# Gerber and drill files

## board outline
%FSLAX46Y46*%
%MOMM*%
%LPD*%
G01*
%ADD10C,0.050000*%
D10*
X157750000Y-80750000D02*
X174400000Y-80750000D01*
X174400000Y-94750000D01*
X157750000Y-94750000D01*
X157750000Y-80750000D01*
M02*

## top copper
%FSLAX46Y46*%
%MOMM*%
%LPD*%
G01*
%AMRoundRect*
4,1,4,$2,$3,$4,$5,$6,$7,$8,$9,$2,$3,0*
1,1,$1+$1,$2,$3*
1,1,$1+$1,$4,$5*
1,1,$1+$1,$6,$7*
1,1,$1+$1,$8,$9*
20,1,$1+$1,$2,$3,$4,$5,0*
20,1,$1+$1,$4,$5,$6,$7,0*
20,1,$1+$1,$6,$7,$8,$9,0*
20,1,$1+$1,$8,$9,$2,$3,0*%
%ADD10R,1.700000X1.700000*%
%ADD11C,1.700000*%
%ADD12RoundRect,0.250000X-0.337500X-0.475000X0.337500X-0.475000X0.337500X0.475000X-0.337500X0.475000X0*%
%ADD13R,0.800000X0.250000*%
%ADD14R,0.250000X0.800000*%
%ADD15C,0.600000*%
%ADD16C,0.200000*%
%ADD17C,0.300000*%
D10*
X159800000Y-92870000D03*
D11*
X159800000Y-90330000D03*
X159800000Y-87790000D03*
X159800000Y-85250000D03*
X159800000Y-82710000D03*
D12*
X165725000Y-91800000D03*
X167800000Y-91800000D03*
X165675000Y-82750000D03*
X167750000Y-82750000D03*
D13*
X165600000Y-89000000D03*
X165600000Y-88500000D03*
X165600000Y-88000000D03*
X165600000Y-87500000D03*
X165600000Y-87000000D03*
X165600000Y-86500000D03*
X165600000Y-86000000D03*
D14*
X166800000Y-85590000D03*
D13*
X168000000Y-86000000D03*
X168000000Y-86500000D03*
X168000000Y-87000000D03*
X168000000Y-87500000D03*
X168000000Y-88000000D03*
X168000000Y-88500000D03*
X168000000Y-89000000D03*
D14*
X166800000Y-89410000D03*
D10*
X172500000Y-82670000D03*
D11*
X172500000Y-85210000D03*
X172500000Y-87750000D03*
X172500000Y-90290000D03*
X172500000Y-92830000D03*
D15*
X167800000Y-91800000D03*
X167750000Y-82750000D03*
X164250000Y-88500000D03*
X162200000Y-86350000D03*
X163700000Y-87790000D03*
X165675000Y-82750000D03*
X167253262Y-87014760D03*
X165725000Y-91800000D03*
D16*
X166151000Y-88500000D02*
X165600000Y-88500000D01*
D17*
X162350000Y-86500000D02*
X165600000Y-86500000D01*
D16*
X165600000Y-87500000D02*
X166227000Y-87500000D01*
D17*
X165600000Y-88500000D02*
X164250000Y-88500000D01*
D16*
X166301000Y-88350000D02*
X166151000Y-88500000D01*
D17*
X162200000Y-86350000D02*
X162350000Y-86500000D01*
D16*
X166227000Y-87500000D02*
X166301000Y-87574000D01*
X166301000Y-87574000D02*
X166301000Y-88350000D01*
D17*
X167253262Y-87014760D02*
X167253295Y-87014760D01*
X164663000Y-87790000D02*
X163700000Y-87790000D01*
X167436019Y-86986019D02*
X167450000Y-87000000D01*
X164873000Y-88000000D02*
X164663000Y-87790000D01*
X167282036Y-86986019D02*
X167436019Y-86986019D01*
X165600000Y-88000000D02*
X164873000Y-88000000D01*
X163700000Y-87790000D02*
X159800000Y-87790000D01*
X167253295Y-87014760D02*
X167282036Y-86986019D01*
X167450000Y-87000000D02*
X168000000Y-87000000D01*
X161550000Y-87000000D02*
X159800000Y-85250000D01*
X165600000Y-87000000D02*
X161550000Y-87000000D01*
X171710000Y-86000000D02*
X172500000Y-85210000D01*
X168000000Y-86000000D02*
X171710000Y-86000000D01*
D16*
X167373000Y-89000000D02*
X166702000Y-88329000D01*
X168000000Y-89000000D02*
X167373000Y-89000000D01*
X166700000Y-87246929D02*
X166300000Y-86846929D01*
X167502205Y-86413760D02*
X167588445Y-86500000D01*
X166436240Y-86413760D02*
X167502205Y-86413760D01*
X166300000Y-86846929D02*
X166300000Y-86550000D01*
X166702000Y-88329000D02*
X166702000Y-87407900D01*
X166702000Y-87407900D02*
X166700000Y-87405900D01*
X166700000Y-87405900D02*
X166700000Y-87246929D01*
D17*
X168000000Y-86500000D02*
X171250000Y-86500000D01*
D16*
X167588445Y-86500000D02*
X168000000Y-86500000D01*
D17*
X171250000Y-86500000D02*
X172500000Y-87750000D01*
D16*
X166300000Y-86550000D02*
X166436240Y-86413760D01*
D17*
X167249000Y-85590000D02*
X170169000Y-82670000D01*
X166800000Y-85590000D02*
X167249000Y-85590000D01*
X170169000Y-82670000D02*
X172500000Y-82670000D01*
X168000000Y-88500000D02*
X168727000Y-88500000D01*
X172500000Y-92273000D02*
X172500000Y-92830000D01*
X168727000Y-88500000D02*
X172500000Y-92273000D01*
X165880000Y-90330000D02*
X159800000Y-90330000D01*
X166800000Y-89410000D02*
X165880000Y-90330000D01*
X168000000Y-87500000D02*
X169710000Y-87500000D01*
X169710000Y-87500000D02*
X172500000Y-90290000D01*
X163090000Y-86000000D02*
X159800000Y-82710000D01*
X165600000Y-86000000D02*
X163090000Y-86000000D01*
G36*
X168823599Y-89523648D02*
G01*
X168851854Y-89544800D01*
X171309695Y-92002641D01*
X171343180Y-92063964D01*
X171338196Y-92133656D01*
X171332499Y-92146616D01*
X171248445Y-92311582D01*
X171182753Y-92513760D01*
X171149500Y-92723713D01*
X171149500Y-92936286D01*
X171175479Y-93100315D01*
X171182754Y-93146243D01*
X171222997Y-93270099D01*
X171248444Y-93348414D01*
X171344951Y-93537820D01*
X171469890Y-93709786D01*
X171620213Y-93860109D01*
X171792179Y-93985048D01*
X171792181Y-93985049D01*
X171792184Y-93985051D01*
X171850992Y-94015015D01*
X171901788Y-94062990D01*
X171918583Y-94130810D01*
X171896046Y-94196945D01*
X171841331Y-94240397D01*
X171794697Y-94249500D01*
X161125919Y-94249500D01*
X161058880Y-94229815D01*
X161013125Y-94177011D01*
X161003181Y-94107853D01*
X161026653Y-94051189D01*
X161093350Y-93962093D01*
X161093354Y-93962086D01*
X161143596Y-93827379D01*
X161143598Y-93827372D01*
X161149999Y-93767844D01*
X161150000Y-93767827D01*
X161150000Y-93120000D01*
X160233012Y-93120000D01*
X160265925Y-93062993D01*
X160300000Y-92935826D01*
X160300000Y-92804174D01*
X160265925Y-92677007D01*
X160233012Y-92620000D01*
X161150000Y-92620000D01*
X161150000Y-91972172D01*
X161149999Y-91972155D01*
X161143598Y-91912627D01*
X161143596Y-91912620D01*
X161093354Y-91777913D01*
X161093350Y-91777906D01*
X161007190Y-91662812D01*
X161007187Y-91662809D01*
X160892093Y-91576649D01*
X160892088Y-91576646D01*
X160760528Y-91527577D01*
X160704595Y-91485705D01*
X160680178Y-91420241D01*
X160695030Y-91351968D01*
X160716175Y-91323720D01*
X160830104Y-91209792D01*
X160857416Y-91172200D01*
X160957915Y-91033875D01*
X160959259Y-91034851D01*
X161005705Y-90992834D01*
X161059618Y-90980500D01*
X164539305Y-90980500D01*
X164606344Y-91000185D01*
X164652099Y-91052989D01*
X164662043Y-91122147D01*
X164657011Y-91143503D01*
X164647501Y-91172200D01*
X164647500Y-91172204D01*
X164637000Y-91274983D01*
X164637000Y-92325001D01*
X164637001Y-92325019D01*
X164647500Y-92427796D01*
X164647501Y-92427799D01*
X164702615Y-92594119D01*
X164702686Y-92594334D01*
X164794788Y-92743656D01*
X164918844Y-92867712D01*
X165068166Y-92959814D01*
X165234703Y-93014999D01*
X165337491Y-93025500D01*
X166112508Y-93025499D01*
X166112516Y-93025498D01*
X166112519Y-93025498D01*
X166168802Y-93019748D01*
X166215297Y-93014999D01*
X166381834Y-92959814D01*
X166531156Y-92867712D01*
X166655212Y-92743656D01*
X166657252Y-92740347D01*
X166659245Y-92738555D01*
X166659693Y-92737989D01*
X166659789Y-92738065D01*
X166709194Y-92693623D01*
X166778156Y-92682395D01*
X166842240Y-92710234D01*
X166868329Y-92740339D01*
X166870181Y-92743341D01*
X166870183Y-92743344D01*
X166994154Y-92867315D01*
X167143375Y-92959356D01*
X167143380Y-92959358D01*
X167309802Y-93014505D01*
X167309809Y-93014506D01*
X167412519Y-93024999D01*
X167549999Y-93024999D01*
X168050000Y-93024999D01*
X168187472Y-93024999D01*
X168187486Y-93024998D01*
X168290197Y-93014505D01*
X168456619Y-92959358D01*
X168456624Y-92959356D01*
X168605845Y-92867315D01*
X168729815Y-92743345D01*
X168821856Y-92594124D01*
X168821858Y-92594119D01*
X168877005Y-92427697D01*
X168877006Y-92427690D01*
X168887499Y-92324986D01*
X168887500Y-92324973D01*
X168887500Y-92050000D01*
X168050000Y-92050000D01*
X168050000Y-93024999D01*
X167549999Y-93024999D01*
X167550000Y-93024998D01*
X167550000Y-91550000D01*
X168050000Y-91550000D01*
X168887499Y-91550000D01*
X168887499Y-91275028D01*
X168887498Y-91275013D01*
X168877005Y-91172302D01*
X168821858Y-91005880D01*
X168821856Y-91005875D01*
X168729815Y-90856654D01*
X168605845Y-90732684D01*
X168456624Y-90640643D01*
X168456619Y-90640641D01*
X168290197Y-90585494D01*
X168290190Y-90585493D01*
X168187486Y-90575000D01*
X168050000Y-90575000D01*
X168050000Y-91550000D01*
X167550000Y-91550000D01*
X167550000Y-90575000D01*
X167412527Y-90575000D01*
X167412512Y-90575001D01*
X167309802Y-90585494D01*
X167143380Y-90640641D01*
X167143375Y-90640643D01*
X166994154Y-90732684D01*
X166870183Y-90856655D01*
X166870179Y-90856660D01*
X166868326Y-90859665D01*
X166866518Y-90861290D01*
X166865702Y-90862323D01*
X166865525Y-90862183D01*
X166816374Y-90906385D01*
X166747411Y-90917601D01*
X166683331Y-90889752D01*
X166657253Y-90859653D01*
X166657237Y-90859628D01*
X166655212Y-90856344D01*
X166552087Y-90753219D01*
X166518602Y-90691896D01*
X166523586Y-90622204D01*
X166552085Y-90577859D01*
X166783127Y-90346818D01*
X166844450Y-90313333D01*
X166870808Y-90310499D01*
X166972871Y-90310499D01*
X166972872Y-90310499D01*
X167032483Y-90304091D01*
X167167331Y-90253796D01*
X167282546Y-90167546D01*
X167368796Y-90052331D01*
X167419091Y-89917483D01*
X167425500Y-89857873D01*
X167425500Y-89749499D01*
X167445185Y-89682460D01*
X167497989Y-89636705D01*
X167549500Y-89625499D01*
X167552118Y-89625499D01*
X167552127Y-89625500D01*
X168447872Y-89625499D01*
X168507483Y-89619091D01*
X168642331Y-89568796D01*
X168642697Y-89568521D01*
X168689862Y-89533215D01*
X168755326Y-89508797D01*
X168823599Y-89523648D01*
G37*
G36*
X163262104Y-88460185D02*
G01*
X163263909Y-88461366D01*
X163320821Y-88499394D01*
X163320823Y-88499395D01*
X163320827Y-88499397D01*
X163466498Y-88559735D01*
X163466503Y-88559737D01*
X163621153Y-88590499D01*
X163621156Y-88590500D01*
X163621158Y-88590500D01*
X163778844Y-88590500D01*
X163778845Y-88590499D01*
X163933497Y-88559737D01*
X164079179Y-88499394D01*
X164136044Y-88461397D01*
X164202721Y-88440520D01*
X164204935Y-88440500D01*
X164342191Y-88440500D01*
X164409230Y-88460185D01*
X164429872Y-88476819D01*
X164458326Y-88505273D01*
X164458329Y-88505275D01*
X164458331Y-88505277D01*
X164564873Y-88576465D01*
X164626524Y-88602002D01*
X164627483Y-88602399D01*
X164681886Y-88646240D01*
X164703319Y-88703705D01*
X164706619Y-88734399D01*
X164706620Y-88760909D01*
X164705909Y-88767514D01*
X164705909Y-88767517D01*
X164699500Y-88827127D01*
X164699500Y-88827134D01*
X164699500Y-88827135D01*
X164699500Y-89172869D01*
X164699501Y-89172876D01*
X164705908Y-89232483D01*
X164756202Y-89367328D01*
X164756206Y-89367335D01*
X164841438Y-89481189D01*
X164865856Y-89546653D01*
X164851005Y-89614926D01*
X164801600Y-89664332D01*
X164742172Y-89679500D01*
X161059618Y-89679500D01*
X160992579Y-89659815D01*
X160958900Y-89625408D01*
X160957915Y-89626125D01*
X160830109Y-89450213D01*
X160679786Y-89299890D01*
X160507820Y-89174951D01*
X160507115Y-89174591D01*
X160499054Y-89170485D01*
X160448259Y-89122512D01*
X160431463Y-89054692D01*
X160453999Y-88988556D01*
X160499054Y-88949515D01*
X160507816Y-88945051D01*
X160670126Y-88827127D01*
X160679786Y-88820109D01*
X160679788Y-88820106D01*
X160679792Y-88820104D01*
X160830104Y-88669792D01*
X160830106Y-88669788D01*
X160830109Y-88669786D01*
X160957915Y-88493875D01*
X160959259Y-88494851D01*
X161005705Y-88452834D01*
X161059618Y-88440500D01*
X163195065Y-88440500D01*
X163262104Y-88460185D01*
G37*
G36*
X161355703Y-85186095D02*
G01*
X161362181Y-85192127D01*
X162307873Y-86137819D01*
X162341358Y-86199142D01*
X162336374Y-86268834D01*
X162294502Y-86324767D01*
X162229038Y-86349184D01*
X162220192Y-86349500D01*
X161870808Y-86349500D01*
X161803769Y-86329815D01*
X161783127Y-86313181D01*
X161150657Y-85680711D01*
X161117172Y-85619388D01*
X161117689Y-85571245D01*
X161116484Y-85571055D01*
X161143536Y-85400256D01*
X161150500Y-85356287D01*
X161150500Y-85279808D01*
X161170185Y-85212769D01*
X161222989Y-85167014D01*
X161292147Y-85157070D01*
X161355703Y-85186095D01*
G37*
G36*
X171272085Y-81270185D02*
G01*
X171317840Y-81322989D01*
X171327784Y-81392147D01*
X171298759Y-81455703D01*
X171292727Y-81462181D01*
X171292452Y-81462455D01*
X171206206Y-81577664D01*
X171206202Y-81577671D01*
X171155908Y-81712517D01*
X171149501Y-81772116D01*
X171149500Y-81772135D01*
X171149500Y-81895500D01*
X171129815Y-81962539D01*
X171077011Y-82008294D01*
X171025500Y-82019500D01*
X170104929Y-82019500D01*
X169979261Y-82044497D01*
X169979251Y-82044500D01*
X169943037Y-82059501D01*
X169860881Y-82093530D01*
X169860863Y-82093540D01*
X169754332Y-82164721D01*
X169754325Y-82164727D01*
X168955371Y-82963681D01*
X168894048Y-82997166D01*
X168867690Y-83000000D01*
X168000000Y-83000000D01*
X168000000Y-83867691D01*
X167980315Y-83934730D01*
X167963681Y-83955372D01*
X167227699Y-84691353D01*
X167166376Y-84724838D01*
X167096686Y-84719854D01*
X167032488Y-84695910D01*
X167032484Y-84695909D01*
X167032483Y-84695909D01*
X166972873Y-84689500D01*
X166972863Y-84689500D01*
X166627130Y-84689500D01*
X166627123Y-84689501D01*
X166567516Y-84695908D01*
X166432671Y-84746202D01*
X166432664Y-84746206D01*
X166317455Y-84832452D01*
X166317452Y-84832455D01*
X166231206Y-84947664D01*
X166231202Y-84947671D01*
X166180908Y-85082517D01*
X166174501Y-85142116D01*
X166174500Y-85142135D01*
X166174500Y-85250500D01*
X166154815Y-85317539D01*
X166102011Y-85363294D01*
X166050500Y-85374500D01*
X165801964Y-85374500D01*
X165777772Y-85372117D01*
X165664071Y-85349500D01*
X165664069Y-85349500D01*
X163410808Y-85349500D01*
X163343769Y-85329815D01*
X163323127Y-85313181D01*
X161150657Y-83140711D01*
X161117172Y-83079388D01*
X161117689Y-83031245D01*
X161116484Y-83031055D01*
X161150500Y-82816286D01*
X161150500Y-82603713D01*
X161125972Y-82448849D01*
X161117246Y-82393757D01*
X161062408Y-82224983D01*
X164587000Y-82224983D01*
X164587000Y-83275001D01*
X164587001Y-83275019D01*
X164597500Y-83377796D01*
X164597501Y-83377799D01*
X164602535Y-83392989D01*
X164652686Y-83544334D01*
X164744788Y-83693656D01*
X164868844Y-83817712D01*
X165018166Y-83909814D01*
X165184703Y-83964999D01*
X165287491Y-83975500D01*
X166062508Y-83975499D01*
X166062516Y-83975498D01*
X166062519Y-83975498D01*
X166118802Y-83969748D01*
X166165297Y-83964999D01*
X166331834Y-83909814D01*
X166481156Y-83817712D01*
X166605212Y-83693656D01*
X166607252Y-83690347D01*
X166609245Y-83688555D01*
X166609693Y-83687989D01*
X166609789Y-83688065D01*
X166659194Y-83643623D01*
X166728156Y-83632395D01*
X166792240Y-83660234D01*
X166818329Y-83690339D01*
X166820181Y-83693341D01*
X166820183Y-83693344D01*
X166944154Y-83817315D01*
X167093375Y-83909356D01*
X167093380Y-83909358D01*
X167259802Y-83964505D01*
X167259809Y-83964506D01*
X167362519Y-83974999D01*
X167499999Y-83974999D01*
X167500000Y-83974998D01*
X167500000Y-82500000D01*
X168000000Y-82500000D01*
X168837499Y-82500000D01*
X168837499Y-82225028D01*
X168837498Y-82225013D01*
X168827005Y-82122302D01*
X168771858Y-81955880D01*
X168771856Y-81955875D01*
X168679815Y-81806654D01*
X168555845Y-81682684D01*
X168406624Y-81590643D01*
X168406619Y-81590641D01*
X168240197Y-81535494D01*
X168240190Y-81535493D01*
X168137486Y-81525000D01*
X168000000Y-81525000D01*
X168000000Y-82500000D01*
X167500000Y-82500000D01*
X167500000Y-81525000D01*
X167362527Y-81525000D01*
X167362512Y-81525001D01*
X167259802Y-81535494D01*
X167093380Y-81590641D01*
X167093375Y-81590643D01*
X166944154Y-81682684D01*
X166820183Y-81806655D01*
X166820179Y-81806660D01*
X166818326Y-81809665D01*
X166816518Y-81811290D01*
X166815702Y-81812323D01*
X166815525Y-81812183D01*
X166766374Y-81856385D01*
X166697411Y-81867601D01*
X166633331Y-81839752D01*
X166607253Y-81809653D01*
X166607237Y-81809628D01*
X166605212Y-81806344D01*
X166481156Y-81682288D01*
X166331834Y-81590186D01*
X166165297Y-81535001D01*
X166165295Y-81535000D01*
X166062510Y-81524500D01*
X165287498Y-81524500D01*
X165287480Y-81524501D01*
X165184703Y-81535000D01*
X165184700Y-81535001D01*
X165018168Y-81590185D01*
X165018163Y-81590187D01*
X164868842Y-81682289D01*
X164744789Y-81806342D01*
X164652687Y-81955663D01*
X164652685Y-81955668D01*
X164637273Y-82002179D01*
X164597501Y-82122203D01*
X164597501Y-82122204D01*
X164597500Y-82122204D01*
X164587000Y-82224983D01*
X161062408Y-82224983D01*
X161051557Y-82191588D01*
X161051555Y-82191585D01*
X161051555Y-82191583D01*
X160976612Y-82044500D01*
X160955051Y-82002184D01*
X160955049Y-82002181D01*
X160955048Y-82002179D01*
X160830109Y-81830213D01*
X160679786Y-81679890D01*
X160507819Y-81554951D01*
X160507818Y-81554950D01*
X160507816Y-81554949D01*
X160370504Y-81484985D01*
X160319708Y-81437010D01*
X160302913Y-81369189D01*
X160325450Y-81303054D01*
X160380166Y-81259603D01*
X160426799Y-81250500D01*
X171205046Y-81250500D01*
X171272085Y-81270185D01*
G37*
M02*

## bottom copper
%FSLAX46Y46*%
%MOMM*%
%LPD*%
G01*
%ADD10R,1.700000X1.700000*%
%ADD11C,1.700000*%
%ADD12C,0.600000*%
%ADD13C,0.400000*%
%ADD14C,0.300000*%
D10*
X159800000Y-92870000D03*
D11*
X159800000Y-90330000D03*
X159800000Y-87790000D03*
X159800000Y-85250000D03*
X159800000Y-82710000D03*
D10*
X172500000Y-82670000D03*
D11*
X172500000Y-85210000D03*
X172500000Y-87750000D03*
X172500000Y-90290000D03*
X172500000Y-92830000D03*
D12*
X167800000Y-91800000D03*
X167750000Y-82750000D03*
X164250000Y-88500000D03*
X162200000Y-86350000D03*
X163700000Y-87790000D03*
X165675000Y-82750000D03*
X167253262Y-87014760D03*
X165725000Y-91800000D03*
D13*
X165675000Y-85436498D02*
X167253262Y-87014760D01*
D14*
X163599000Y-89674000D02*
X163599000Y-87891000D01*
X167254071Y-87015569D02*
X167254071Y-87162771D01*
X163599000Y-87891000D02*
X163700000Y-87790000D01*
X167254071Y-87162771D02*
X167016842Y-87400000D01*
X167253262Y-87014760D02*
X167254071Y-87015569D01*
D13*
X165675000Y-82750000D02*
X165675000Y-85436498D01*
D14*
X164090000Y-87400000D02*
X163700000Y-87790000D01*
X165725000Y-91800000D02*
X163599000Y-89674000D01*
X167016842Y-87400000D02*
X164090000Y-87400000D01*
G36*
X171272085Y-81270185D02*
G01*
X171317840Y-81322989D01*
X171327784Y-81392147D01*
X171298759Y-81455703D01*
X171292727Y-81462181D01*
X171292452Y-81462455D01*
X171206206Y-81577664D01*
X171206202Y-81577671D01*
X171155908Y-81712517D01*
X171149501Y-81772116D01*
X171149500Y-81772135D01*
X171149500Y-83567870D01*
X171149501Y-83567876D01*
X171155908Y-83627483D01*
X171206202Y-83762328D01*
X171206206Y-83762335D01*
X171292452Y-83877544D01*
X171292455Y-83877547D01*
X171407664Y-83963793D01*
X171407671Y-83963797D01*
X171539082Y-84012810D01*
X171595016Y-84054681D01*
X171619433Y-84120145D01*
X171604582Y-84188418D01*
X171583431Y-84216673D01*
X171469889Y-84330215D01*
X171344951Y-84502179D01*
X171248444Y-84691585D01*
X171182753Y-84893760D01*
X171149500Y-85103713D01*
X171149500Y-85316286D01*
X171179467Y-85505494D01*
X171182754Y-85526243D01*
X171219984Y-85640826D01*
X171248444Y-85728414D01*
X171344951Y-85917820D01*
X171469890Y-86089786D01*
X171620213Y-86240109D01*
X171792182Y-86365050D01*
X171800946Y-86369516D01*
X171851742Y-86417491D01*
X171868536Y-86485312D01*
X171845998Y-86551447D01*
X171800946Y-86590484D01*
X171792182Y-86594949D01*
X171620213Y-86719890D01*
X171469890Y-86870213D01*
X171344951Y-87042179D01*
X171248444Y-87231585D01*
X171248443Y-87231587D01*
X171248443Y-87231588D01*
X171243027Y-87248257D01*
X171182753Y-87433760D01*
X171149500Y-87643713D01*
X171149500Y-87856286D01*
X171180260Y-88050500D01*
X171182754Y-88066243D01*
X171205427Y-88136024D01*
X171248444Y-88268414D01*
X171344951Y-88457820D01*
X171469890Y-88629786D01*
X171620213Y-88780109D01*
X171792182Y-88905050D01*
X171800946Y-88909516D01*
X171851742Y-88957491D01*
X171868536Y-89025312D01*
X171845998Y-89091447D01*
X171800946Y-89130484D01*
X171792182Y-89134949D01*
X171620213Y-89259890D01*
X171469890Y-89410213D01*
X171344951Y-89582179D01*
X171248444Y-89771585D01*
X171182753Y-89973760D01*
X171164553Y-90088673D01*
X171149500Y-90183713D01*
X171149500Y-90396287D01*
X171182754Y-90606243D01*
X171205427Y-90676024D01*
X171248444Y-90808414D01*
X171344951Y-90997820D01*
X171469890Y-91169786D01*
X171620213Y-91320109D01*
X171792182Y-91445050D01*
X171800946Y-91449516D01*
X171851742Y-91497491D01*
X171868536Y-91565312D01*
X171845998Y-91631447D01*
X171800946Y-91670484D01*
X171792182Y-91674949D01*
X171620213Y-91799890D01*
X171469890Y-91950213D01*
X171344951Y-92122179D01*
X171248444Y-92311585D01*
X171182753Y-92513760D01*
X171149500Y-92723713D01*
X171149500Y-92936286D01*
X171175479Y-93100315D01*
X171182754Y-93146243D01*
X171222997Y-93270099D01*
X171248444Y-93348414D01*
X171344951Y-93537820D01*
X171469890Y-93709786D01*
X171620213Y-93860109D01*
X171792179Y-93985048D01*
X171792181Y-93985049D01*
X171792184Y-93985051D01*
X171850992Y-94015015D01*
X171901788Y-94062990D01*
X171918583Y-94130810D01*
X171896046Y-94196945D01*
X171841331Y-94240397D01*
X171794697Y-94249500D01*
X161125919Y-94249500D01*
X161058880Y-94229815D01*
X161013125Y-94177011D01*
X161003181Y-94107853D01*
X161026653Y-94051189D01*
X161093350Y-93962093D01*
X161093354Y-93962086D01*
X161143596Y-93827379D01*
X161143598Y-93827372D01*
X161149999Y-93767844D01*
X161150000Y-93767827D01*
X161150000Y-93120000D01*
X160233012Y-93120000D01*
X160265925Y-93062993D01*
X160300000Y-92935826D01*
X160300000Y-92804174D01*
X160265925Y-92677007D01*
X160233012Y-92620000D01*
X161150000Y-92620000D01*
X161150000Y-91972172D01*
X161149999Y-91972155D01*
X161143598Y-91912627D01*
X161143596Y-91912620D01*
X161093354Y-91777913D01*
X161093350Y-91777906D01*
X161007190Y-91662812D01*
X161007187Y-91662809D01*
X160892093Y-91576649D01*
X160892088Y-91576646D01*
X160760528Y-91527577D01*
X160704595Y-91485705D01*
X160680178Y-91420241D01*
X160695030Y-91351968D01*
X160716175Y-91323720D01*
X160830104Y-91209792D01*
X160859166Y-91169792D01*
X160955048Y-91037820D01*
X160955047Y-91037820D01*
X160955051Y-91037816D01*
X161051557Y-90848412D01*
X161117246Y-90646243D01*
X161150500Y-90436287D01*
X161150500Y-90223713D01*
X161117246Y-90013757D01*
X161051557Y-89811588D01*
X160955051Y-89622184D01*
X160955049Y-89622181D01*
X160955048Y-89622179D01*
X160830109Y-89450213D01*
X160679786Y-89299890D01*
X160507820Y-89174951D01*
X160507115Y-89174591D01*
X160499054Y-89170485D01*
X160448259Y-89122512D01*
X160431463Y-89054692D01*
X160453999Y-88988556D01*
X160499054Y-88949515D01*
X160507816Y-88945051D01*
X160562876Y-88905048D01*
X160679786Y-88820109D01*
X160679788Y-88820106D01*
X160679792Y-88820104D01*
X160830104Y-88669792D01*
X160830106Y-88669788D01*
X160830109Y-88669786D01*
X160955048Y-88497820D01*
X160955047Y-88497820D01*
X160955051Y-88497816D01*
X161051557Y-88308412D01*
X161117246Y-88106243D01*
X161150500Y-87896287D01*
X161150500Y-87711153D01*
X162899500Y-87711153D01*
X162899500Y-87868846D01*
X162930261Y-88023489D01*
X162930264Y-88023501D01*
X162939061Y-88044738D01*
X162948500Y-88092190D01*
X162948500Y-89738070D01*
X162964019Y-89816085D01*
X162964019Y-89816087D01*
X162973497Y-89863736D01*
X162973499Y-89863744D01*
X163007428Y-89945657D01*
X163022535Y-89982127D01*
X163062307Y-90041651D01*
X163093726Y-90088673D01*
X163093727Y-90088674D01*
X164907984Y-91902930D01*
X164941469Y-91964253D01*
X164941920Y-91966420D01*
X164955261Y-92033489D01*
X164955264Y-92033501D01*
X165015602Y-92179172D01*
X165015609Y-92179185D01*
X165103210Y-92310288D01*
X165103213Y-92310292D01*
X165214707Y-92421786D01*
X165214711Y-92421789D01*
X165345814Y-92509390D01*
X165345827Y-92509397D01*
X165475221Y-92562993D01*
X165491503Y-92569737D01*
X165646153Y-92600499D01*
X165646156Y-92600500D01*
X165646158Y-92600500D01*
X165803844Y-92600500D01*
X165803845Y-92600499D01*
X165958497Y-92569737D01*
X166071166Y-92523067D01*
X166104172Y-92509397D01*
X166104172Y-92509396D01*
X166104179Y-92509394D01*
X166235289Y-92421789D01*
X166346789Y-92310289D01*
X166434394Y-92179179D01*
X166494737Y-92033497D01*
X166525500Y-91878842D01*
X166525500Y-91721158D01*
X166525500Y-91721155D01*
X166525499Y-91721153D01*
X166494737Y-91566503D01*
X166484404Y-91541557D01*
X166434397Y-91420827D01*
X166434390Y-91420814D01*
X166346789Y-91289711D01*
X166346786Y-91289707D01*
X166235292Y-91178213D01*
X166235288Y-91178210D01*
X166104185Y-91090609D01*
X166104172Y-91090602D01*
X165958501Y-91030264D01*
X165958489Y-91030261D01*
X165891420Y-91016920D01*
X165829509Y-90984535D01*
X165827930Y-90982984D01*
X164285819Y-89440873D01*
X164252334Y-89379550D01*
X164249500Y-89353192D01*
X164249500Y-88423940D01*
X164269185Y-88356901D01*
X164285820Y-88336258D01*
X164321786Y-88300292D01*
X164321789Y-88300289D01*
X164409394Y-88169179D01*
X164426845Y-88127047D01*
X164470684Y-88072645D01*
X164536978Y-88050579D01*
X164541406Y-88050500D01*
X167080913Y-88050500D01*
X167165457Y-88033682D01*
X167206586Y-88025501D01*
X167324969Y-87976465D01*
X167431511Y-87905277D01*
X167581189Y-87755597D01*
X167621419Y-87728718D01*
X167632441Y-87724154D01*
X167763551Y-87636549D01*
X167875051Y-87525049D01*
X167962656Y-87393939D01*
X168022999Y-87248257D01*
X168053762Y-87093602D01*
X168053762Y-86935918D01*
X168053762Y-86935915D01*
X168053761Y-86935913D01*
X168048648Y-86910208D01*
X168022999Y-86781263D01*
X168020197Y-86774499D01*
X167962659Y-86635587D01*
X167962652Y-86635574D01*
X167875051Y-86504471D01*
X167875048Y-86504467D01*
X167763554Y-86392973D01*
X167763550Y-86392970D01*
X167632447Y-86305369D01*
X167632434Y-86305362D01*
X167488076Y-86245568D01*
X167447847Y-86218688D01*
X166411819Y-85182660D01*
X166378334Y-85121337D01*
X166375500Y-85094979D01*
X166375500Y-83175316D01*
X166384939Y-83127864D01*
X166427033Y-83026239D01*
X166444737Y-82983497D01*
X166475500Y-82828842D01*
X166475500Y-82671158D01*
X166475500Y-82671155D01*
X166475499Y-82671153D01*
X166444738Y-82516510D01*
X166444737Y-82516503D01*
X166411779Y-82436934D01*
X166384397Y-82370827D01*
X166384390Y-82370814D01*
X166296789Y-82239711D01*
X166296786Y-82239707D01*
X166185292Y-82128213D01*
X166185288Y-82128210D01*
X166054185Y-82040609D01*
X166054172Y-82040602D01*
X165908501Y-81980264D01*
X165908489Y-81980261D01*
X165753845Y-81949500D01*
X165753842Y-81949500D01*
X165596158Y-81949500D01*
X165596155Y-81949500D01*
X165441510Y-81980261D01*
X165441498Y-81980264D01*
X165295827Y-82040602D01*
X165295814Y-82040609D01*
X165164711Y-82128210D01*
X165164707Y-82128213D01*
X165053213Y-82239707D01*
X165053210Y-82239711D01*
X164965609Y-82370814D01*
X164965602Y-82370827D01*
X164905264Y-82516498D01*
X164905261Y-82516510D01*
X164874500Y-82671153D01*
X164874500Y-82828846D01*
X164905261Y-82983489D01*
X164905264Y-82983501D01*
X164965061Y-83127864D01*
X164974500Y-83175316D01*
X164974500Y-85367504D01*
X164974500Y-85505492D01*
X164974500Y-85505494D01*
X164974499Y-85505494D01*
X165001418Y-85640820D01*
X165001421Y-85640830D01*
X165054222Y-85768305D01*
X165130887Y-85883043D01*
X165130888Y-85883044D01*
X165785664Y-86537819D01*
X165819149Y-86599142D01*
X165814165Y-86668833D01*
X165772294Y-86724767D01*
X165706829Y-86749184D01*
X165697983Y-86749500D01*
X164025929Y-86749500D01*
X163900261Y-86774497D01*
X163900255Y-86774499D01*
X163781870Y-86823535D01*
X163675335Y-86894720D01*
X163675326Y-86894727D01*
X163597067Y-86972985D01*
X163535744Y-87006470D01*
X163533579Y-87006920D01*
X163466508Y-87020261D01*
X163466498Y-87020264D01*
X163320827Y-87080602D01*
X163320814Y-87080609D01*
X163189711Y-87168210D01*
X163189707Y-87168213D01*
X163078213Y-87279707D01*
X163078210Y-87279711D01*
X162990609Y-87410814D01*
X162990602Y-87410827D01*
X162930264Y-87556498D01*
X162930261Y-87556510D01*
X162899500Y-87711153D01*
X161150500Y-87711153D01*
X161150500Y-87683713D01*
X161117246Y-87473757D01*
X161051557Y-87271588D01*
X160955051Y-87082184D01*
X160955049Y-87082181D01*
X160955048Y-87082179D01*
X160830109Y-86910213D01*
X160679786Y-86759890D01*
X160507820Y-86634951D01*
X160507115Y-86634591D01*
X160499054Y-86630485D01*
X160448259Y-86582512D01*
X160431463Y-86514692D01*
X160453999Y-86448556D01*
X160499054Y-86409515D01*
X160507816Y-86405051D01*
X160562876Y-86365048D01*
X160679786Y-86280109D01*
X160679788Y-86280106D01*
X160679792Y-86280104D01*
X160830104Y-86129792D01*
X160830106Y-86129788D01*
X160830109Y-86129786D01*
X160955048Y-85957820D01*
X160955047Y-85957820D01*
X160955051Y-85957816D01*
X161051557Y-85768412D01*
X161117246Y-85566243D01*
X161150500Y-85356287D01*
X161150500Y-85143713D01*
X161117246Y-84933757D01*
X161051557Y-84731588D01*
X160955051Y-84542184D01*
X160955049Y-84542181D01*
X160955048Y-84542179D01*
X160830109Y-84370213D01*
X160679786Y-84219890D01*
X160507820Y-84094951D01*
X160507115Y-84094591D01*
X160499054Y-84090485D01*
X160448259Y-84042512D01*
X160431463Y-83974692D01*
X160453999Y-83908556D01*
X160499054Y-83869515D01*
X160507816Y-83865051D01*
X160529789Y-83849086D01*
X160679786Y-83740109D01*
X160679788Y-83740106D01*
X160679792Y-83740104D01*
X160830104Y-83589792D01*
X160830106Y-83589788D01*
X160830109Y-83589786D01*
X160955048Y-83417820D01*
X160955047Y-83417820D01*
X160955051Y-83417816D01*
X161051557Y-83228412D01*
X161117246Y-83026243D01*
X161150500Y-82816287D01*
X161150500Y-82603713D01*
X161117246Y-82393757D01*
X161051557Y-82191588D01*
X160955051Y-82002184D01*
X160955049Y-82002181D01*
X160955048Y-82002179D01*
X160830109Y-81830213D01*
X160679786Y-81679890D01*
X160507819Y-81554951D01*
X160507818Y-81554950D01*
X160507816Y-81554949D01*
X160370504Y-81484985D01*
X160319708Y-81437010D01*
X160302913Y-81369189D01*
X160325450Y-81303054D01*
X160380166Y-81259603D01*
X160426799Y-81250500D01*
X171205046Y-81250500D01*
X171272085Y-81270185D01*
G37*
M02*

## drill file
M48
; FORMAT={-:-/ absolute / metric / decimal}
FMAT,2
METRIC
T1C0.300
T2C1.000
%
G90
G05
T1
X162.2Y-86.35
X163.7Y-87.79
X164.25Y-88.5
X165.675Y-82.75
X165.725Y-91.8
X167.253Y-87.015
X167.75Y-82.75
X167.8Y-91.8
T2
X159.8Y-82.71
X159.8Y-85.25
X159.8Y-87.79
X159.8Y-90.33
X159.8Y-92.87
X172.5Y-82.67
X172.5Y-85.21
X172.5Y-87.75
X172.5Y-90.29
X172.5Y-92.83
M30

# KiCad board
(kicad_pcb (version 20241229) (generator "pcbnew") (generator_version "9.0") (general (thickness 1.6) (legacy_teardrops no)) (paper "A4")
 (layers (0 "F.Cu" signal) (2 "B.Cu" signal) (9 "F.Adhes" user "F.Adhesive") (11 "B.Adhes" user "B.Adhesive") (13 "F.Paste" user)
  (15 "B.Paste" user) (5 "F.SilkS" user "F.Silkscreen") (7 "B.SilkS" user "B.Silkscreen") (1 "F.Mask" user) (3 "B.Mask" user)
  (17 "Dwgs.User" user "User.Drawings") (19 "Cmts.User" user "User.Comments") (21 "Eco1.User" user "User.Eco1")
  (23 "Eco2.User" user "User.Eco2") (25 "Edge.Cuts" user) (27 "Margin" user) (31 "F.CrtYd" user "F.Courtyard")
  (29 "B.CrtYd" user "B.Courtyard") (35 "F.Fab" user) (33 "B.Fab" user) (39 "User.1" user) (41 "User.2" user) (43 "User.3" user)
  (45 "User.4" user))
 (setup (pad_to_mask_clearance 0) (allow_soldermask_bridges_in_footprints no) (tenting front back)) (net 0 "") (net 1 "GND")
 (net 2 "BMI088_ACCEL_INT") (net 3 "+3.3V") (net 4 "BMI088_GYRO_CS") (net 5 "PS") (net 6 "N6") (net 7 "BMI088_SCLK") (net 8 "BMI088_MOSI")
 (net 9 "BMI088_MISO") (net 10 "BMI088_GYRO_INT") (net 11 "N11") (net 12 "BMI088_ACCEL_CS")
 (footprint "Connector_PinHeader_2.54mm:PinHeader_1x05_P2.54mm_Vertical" (layer "F.Cu") (at 159.8 92.87 180)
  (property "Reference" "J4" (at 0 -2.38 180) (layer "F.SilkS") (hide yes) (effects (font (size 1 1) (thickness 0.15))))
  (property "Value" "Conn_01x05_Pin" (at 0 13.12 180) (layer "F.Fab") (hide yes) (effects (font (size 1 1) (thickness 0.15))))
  (pad "1" thru_hole rect (at 0 0 180) (size 1.7 1.7) (drill 1) (layers "*.Cu" "*.Mask") (remove_unused_layers no) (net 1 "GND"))
  (pad "2" thru_hole circle (at 0 2.54 180) (size 1.7 1.7) (drill 1) (layers "*.Cu" "*.Mask") (remove_unused_layers no)
   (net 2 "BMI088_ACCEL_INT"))
  (pad "3" thru_hole circle (at 0 5.08 180) (size 1.7 1.7) (drill 1) (layers "*.Cu" "*.Mask") (remove_unused_layers no) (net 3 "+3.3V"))
  (pad "4" thru_hole circle (at 0 7.62 180) (size 1.7 1.7) (drill 1) (layers "*.Cu" "*.Mask") (remove_unused_layers no)
   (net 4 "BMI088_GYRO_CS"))
  (pad "5" thru_hole circle (at 0 10.16 180) (size 1.7 1.7) (drill 1) (layers "*.Cu" "*.Mask") (remove_unused_layers no) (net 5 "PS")))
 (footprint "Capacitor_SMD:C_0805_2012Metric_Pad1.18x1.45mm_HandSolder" (layer "F.Cu") (at 166.7625 91.8)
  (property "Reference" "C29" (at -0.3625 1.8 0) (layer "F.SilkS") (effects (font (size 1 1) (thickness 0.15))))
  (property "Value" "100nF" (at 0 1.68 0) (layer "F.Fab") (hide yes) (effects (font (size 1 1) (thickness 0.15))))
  (pad "1" smd roundrect (at -1.0375 0) (size 1.175 1.45) (layers "F.Cu" "F.Mask" "F.Paste") (roundrect_rratio 0.212766) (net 3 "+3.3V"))
  (pad "2" smd roundrect (at 1.0375 0) (size 1.175 1.45) (layers "F.Cu" "F.Mask" "F.Paste") (roundrect_rratio 0.212766) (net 1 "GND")))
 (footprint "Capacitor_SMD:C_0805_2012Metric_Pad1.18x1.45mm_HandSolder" (layer "F.Cu") (at 166.7125 82.75)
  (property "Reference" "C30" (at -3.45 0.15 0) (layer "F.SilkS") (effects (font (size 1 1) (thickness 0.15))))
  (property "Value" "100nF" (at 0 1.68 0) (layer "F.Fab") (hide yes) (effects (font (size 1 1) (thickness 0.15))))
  (pad "1" smd roundrect (at -1.0375 0) (size 1.175 1.45) (layers "F.Cu" "F.Mask" "F.Paste") (roundrect_rratio 0.212766) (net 3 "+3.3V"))
  (pad "2" smd roundrect (at 1.0375 0) (size 1.175 1.45) (layers "F.Cu" "F.Mask" "F.Paste") (roundrect_rratio 0.212766) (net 1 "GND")))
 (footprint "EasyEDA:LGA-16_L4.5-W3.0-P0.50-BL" (layer "F.Cu") (at 166.8 87.5)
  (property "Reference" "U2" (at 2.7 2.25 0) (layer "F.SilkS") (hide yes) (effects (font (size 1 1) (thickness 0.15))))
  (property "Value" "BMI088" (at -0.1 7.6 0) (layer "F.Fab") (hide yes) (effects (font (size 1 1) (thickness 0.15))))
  (pad "1" smd rect (at -1.2 1.5 90) (size 0.25 0.8) (layers "F.Cu" "F.Mask" "F.Paste") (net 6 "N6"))
  (pad "2" smd rect (at -1.2 1 90) (size 0.25 0.8) (layers "F.Cu" "F.Mask" "F.Paste") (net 1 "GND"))
  (pad "3" smd rect (at -1.2 0.5 90) (size 0.25 0.8) (layers "F.Cu" "F.Mask" "F.Paste") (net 3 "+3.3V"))
  (pad "4" smd rect (at -1.2 0 90) (size 0.25 0.8) (layers "F.Cu" "F.Mask" "F.Paste") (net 1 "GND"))
  (pad "5" smd rect (at -1.2 -0.5 90) (size 0.25 0.8) (layers "F.Cu" "F.Mask" "F.Paste") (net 4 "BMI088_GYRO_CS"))
  (pad "6" smd rect (at -1.2 -1 90) (size 0.25 0.8) (layers "F.Cu" "F.Mask" "F.Paste") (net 1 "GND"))
  (pad "7" smd rect (at -1.2 -1.5 90) (size 0.25 0.8) (layers "F.Cu" "F.Mask" "F.Paste") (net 5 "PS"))
  (pad "8" smd rect (at 0 -1.91 180) (size 0.25 0.8) (layers "F.Cu" "F.Mask" "F.Paste") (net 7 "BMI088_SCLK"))
  (pad "9" smd rect (at 1.2 -1.5 270) (size 0.25 0.8) (layers "F.Cu" "F.Mask" "F.Paste") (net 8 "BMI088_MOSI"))
  (pad "10" smd rect (at 1.2 -1 270) (size 0.25 0.8) (layers "F.Cu" "F.Mask" "F.Paste") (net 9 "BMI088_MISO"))
  (pad "11" smd rect (at 1.2 -0.5 270) (size 0.25 0.8) (layers "F.Cu" "F.Mask" "F.Paste") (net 3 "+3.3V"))
  (pad "12" smd rect (at 1.2 0 270) (size 0.25 0.8) (layers "F.Cu" "F.Mask" "F.Paste") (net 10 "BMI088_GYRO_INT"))
  (pad "13" smd rect (at 1.2 0.5 270) (size 0.25 0.8) (layers "F.Cu" "F.Mask" "F.Paste") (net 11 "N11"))
  (pad "14" smd rect (at 1.2 1 270) (size 0.25 0.8) (layers "F.Cu" "F.Mask" "F.Paste") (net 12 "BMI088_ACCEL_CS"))
  (pad "15" smd rect (at 1.2 1.5 270) (size 0.25 0.8) (layers "F.Cu" "F.Mask" "F.Paste") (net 9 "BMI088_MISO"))
  (pad "16" smd rect (at 0 1.91) (size 0.25 0.8) (layers "F.Cu" "F.Mask" "F.Paste") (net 2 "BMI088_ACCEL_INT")))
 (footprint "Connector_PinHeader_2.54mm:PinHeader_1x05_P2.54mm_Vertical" (layer "B.Cu") (at 172.5 82.67 180)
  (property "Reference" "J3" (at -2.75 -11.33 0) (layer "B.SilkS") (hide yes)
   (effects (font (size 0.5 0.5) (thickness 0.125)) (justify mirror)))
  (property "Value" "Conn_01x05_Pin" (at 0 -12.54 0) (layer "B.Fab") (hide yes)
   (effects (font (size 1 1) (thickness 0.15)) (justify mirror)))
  (pad "1" thru_hole rect (at 0 0 180) (size 1.7 1.7) (drill 1) (layers "*.Cu" "*.Mask") (remove_unused_layers no) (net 7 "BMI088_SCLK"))
  (pad "2" thru_hole circle (at 0 -2.54 180) (size 1.7 1.7) (drill 1) (layers "*.Cu" "*.Mask") (remove_unused_layers no)
   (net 8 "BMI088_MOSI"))
  (pad "3" thru_hole circle (at 0 -5.08 180) (size 1.7 1.7) (drill 1) (layers "*.Cu" "*.Mask") (remove_unused_layers no)
   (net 9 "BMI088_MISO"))
  (pad "4" thru_hole circle (at 0 -7.62 180) (size 1.7 1.7) (drill 1) (layers "*.Cu" "*.Mask") (remove_unused_layers no)
   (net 10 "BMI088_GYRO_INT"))
  (pad "5" thru_hole circle (at 0 -10.16 180) (size 1.7 1.7) (drill 1) (layers "*.Cu" "*.Mask") (remove_unused_layers no)
   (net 12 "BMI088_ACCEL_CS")))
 (gr_rect (start 157.75 80.75) (end 174.4 94.75) (stroke (width 0.05) (type default)) (fill no) (layer "Edge.Cuts"))
 (segment (start 166.151 88.5) (end 165.6 88.5) (width 0.2) (layer "F.Cu") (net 1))
 (segment (start 162.35 86.5) (end 165.6 86.5) (width 0.3) (layer "F.Cu") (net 1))
 (segment (start 165.6 87.5) (end 166.227 87.5) (width 0.2) (layer "F.Cu") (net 1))
 (segment (start 165.6 88.5) (end 164.25 88.5) (width 0.3) (layer "F.Cu") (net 1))
 (segment (start 166.301 88.35) (end 166.151 88.5) (width 0.2) (layer "F.Cu") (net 1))
 (segment (start 162.2 86.35) (end 162.35 86.5) (width 0.3) (layer "F.Cu") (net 1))
 (segment (start 166.227 87.5) (end 166.301 87.574) (width 0.2) (layer "F.Cu") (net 1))
 (segment (start 166.301 87.574) (end 166.301 88.35) (width 0.2) (layer "F.Cu") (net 1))
 (via (at 167.8 91.8) (size 0.6) (drill 0.3) (layers "F.Cu" "B.Cu") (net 1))
 (via (at 167.75 82.75) (size 0.6) (drill 0.3) (layers "F.Cu" "B.Cu") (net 1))
 (via (at 164.25 88.5) (size 0.6) (drill 0.3) (layers "F.Cu" "B.Cu") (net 1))
 (via (at 162.2 86.35) (size 0.6) (drill 0.3) (layers "F.Cu" "B.Cu") (free yes) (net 1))
 (segment (start 167.253262 87.01476) (end 167.253295 87.01476) (width 0.3) (layer "F.Cu") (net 3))
 (segment (start 164.663 87.79) (end 163.7 87.79) (width 0.3) (layer "F.Cu") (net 3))
 (segment (start 167.436019 86.986019) (end 167.45 87) (width 0.3) (layer "F.Cu") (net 3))
 (segment (start 164.873 88) (end 164.663 87.79) (width 0.3) (layer "F.Cu") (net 3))
 (segment (start 167.282036 86.986019) (end 167.436019 86.986019) (width 0.3) (layer "F.Cu") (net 3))
 (segment (start 165.6 88) (end 164.873 88) (width 0.3) (layer "F.Cu") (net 3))
 (segment (start 163.7 87.79) (end 159.8 87.79) (width 0.3) (layer "F.Cu") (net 3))
 (segment (start 167.253295 87.01476) (end 167.282036 86.986019) (width 0.3) (layer "F.Cu") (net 3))
 (segment (start 167.45 87) (end 168 87) (width 0.3) (layer "F.Cu") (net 3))
 (via (at 163.7 87.79) (size 0.6) (drill 0.3) (layers "F.Cu" "B.Cu") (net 3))
 (via (at 165.675 82.75) (size 0.6) (drill 0.3) (layers "F.Cu" "B.Cu") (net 3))
 (via (at 167.253262 87.01476) (size 0.6) (drill 0.3) (layers "F.Cu" "B.Cu") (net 3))
 (via (at 165.725 91.8) (size 0.6) (drill 0.3) (layers "F.Cu" "B.Cu") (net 3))
 (segment (start 165.675 85.436498) (end 167.253262 87.01476) (width 0.4) (layer "B.Cu") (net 3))
 (segment (start 163.599 89.674) (end 163.599 87.891) (width 0.3) (layer "B.Cu") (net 3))
 (segment (start 167.254071 87.015569) (end 167.254071 87.162771) (width 0.3) (layer "B.Cu") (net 3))
 (segment (start 163.599 87.891) (end 163.7 87.79) (width 0.3) (layer "B.Cu") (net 3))
 (segment (start 167.254071 87.162771) (end 167.016842 87.4) (width 0.3) (layer "B.Cu") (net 3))
 (segment (start 167.253262 87.01476) (end 167.254071 87.015569) (width 0.3) (layer "B.Cu") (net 3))
 (segment (start 165.675 82.75) (end 165.675 85.436498) (width 0.4) (layer "B.Cu") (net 3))
 (segment (start 164.09 87.4) (end 163.7 87.79) (width 0.3) (layer "B.Cu") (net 3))
 (segment (start 165.725 91.8) (end 163.599 89.674) (width 0.3) (layer "B.Cu") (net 3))
 (segment (start 167.016842 87.4) (end 164.09 87.4) (width 0.3) (layer "B.Cu") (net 3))
 (segment (start 161.55 87) (end 159.8 85.25) (width 0.3) (layer "F.Cu") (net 4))
 (segment (start 165.6 87) (end 161.55 87) (width 0.3) (layer "F.Cu") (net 4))
 (segment (start 171.71 86) (end 172.5 85.21) (width 0.3) (layer "F.Cu") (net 8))
 (segment (start 168 86) (end 171.71 86) (width 0.3) (layer "F.Cu") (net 8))
 (segment (start 167.373 89) (end 166.702 88.329) (width 0.2) (layer "F.Cu") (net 9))
 (segment (start 168 89) (end 167.373 89) (width 0.2) (layer "F.Cu") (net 9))
 (segment (start 166.7 87.246929) (end 166.3 86.846929) (width 0.2) (layer "F.Cu") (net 9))
 (segment (start 167.502205 86.41376) (end 167.588445 86.5) (width 0.2) (layer "F.Cu") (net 9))
 (segment (start 166.43624 86.41376) (end 167.502205 86.41376) (width 0.2) (layer "F.Cu") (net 9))
 (segment (start 166.3 86.846929) (end 166.3 86.55) (width 0.2) (layer "F.Cu") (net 9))
 (segment (start 166.702 88.329) (end 166.702 87.4079) (width 0.2) (layer "F.Cu") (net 9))
 (segment (start 166.702 87.4079) (end 166.7 87.4059) (width 0.2) (layer "F.Cu") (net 9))
 (segment (start 166.7 87.4059) (end 166.7 87.246929) (width 0.2) (layer "F.Cu") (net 9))
 (segment (start 168 86.5) (end 171.25 86.5) (width 0.3) (layer "F.Cu") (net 9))
 (segment (start 167.588445 86.5) (end 168 86.5) (width 0.2) (layer "F.Cu") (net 9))
 (segment (start 171.25 86.5) (end 172.5 87.75) (width 0.3) (layer "F.Cu") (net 9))
 (segment (start 166.3 86.55) (end 166.43624 86.41376) (width 0.2) (layer "F.Cu") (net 9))
 (segment (start 167.249 85.59) (end 170.169 82.67) (width 0.3) (layer "F.Cu") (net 7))
 (segment (start 166.8 85.59) (end 167.249 85.59) (width 0.3) (layer "F.Cu") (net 7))
 (segment (start 170.169 82.67) (end 172.5 82.67) (width 0.3) (layer "F.Cu") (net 7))
 (segment (start 168 88.5) (end 168.727 88.5) (width 0.3) (layer "F.Cu") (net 12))
 (segment (start 172.5 92.273) (end 172.5 92.83) (width 0.3) (layer "F.Cu") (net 12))
 (segment (start 168.727 88.5) (end 172.5 92.273) (width 0.3) (layer "F.Cu") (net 12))
 (segment (start 165.88 90.33) (end 159.8 90.33) (width 0.3) (layer "F.Cu") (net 2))
 (segment (start 166.8 89.41) (end 165.88 90.33) (width 0.3) (layer "F.Cu") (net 2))
 (segment (start 168 87.5) (end 169.71 87.5) (width 0.3) (layer "F.Cu") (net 10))
 (segment (start 169.71 87.5) (end 172.5 90.29) (width 0.3) (layer "F.Cu") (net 10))
 (segment (start 163.09 86) (end 159.8 82.71) (width 0.3) (layer "F.Cu") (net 5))
 (segment (start 165.6 86) (end 163.09 86) (width 0.3) (layer "F.Cu") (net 5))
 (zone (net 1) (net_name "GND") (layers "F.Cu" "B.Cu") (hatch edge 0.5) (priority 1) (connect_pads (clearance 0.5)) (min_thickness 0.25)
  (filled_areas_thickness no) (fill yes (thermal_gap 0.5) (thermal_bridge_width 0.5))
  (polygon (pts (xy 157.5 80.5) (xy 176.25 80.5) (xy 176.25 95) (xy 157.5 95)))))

